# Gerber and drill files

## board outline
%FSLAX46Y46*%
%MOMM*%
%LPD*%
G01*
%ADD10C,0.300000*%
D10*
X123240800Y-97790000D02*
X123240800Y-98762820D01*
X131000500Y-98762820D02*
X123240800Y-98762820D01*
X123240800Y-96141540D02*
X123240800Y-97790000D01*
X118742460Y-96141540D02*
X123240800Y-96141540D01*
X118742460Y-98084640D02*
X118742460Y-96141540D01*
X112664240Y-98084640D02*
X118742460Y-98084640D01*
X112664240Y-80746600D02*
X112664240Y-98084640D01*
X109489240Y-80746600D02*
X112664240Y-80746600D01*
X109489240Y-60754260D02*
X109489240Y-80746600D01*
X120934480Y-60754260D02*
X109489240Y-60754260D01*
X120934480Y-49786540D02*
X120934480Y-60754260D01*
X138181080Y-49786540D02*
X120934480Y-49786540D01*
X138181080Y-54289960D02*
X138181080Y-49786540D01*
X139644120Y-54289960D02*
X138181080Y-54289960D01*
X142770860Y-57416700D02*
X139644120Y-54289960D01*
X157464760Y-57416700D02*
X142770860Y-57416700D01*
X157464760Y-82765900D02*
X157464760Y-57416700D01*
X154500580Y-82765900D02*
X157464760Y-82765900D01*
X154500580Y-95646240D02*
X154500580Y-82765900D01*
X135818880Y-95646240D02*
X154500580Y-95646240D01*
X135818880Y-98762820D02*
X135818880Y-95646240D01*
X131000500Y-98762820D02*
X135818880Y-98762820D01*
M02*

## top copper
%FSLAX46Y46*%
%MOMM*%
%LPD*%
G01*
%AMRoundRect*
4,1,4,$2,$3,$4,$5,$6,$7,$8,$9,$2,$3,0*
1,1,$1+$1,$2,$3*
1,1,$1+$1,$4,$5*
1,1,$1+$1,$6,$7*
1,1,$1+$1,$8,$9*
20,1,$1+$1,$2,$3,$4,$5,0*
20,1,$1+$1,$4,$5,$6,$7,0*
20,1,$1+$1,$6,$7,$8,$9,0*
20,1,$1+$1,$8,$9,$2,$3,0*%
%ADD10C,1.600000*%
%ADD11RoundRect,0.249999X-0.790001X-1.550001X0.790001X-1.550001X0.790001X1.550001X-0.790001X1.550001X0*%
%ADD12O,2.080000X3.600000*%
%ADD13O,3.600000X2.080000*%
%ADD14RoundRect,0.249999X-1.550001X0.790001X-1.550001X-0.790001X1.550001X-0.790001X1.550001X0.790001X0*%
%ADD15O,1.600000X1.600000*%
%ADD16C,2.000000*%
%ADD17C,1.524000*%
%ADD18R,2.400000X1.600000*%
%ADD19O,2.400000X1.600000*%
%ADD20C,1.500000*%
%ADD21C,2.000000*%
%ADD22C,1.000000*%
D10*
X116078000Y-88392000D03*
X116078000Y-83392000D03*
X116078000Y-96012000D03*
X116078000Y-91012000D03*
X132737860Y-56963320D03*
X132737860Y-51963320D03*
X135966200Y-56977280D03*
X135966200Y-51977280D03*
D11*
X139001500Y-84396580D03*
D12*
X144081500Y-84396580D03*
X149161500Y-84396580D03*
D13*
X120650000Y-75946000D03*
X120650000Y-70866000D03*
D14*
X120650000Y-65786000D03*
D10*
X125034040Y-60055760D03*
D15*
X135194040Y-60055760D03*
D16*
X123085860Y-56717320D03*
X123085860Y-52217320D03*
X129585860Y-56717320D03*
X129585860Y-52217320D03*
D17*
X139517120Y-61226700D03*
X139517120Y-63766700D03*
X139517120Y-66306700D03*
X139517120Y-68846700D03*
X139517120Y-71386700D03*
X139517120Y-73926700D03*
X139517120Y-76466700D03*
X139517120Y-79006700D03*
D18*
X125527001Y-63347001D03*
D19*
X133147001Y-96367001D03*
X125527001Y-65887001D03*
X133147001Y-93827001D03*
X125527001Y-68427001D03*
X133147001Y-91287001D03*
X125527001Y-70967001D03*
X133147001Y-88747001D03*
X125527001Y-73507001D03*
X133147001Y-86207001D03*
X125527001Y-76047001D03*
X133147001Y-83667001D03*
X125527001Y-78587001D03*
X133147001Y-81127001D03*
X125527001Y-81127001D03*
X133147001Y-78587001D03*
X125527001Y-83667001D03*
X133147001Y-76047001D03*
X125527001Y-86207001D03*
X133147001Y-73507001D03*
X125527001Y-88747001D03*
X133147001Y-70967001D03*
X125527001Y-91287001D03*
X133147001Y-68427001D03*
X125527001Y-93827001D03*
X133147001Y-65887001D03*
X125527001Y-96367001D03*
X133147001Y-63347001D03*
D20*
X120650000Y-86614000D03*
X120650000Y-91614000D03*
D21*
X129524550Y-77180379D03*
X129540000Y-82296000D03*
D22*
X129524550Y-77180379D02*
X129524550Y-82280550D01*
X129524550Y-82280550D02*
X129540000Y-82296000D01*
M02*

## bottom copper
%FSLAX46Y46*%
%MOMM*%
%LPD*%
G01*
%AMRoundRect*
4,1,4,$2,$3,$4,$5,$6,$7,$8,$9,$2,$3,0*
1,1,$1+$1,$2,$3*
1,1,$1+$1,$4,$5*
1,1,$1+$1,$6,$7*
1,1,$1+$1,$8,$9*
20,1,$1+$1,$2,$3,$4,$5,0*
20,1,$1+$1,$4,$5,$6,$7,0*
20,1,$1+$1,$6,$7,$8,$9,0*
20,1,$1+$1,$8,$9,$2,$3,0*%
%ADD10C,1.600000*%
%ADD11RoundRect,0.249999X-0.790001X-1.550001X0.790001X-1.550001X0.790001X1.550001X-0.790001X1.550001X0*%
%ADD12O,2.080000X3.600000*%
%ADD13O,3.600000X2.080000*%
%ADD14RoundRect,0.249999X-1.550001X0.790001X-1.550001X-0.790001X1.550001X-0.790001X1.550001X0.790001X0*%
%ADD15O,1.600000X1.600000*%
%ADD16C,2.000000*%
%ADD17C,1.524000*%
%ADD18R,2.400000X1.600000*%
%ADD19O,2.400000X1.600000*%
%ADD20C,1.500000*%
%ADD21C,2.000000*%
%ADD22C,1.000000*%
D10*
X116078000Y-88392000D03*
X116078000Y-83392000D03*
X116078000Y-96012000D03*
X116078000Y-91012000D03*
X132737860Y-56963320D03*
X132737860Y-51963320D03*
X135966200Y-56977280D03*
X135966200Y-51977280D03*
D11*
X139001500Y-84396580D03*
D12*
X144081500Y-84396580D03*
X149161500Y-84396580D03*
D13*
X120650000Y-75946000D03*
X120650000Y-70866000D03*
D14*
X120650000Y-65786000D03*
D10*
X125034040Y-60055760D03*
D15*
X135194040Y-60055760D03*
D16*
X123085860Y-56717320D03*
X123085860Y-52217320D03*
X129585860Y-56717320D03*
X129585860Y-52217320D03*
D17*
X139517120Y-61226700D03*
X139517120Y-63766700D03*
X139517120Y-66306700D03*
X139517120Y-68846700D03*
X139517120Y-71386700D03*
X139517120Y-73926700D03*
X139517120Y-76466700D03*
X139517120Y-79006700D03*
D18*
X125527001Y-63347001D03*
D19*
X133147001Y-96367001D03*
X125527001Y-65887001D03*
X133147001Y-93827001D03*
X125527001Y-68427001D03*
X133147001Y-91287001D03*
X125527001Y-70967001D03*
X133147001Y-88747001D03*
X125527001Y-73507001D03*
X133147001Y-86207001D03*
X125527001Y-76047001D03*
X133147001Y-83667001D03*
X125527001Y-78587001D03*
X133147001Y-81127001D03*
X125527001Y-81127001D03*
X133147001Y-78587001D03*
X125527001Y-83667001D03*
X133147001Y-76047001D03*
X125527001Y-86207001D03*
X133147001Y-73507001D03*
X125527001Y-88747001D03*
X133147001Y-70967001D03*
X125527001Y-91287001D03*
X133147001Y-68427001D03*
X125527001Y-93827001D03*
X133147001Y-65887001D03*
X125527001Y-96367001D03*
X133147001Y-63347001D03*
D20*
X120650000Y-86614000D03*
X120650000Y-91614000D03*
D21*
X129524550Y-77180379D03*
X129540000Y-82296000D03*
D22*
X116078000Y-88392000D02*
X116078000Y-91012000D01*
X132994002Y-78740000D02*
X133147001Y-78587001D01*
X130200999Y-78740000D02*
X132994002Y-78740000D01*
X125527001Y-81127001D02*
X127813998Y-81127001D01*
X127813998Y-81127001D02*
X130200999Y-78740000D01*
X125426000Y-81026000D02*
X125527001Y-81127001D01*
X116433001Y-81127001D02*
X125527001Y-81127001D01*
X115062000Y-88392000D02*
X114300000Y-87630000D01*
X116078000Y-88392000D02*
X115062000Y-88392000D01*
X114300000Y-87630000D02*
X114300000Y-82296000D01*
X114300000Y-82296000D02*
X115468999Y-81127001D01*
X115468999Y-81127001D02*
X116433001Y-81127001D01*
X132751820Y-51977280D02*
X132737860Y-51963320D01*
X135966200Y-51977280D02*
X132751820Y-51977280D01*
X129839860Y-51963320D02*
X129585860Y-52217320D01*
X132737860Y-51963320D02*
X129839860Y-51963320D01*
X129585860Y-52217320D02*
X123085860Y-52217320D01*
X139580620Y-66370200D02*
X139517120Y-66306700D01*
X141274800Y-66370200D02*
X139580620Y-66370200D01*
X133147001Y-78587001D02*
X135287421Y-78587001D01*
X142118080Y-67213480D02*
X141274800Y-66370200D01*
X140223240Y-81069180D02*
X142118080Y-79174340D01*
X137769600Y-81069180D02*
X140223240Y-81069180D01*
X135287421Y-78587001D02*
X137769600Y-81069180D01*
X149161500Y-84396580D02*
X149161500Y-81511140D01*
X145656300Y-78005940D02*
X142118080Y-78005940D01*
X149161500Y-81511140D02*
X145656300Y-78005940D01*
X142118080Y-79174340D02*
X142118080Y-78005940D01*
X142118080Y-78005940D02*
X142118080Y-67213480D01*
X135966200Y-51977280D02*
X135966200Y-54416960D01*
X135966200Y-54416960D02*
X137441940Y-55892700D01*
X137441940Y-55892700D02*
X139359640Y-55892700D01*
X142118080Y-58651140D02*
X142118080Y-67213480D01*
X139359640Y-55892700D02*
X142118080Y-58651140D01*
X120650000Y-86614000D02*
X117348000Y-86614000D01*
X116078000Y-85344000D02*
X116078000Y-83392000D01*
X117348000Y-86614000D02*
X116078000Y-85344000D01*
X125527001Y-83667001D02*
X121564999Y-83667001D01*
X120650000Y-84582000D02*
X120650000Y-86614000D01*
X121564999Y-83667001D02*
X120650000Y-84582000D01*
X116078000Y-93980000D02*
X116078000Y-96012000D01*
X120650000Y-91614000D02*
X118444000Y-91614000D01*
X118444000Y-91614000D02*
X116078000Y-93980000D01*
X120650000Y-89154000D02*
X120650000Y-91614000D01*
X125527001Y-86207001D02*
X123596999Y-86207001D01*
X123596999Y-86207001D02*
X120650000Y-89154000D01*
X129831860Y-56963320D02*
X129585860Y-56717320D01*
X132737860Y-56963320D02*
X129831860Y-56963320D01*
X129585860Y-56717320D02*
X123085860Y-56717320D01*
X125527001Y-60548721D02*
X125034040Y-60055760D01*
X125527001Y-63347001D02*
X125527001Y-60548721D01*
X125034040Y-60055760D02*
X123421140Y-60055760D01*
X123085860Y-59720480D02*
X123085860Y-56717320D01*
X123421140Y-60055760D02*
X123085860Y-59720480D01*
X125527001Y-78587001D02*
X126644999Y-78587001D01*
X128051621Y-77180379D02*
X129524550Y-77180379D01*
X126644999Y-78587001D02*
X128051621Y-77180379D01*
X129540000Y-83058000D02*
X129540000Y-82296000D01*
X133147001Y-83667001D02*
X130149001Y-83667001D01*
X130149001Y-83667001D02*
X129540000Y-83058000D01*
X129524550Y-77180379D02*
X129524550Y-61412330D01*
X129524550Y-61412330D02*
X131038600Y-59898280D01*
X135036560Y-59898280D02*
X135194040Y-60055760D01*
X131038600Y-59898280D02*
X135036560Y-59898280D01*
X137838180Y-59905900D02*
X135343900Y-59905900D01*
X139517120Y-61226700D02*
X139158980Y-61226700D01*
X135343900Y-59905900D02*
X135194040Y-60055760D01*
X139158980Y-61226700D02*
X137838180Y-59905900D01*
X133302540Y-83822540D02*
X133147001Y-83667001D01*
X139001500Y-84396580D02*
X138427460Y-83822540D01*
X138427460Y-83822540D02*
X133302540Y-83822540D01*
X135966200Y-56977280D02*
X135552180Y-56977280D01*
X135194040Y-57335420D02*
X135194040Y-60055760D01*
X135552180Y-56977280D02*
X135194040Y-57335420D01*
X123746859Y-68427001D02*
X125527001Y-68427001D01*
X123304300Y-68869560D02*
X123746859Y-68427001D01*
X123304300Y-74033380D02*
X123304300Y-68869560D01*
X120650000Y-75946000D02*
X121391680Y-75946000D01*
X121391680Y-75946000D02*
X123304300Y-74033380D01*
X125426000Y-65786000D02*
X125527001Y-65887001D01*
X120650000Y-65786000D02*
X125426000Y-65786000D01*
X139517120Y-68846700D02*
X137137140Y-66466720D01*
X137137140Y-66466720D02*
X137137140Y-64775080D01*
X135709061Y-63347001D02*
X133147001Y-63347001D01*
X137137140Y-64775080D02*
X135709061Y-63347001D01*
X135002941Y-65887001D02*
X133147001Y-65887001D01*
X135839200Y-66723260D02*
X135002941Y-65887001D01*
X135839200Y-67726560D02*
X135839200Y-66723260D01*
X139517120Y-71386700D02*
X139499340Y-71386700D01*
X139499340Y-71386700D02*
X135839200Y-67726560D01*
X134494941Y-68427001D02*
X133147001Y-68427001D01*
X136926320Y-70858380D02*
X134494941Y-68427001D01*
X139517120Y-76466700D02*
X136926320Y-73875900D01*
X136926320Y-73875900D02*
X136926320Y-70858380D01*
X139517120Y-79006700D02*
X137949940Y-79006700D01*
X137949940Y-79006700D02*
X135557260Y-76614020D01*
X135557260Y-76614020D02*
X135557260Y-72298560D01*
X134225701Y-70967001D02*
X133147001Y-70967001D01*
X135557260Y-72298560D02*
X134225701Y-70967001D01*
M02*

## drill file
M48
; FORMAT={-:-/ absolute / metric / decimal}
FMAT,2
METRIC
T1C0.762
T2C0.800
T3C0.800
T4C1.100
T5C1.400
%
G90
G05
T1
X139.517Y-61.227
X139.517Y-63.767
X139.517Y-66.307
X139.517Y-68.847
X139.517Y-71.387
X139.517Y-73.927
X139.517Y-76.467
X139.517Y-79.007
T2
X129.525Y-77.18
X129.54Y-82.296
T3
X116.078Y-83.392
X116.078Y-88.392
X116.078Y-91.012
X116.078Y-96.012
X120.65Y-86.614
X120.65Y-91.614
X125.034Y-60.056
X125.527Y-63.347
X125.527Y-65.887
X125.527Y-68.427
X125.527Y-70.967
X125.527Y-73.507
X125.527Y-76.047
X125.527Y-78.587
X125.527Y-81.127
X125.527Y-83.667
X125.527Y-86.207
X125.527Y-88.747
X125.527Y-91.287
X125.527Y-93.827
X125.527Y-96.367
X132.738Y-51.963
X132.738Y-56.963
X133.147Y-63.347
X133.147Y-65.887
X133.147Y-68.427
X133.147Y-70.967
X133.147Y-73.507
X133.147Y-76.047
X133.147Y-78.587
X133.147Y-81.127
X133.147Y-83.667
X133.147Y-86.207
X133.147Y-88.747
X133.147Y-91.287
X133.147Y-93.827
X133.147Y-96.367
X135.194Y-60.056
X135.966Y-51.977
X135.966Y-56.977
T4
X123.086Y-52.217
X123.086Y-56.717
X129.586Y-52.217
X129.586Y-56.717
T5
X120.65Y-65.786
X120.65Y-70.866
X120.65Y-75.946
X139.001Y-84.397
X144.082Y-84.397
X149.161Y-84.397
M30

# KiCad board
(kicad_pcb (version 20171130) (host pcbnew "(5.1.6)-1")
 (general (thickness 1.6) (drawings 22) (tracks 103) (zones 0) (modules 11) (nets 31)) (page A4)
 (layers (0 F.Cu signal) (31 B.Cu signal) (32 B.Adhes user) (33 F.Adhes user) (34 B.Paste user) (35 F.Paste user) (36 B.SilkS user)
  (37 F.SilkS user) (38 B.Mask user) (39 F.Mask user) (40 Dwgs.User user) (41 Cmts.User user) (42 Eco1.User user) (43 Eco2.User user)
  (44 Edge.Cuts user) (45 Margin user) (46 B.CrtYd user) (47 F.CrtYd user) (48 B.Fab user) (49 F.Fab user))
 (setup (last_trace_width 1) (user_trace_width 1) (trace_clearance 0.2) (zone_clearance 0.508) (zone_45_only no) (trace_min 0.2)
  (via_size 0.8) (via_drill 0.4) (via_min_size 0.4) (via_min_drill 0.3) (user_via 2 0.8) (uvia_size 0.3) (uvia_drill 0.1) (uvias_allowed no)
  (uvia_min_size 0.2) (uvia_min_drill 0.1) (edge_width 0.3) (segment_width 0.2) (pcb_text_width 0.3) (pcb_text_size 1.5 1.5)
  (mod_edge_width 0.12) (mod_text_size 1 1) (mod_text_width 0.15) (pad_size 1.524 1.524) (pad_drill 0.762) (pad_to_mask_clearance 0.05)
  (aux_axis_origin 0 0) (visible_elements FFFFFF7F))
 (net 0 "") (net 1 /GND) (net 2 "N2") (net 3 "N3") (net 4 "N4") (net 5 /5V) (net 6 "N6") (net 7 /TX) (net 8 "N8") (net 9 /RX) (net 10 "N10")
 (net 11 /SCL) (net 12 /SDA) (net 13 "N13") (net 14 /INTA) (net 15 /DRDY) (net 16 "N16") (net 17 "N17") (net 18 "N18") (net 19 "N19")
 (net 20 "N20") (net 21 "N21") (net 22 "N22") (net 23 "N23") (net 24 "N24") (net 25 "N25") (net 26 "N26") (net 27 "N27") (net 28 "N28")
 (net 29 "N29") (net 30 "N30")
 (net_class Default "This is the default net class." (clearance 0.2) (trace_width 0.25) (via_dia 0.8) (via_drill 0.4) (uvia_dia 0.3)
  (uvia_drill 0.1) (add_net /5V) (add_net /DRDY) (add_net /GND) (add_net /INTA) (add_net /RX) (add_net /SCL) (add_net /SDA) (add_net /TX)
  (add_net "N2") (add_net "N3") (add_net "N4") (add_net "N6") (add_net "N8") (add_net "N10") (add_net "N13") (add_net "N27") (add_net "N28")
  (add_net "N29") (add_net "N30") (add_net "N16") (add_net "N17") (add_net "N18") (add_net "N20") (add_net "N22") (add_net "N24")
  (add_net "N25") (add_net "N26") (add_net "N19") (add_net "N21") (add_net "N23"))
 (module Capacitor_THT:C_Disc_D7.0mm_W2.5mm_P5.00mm (layer F.Cu) (at 116.078 83.392 270)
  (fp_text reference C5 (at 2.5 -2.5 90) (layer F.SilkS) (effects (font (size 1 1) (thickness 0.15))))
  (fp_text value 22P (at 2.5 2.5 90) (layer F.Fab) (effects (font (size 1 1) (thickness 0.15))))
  (pad 2 thru_hole circle (at 5 0 270) (size 1.6 1.6) (drill 0.8) (layers *.Cu *.Mask) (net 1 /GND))
  (pad 1 thru_hole circle (at 0 0 270) (size 1.6 1.6) (drill 0.8) (layers *.Cu *.Mask) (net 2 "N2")))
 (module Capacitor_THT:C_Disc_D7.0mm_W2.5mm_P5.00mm (layer F.Cu) (at 116.078 96.012 90)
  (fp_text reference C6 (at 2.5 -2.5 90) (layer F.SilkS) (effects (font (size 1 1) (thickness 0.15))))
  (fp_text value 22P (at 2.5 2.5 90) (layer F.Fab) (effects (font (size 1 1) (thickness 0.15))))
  (pad 1 thru_hole circle (at 0 0 90) (size 1.6 1.6) (drill 0.8) (layers *.Cu *.Mask) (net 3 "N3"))
  (pad 2 thru_hole circle (at 5 0 90) (size 1.6 1.6) (drill 0.8) (layers *.Cu *.Mask) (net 1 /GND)))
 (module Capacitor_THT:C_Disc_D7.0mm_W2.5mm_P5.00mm (layer F.Cu) (at 132.73786 51.96332 270)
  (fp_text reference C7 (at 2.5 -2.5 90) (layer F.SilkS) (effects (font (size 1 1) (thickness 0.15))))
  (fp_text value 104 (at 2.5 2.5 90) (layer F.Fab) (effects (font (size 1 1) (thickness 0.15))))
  (pad 2 thru_hole circle (at 5 0 270) (size 1.6 1.6) (drill 0.8) (layers *.Cu *.Mask) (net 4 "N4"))
  (pad 1 thru_hole circle (at 0 0 270) (size 1.6 1.6) (drill 0.8) (layers *.Cu *.Mask) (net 1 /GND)))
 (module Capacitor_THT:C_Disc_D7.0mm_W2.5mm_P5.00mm (layer F.Cu) (at 135.9662 56.97728 90)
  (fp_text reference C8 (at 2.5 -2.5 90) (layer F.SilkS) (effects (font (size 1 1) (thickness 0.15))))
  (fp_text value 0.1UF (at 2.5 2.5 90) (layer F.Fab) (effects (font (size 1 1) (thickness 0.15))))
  (pad 1 thru_hole circle (at 0 0 90) (size 1.6 1.6) (drill 0.8) (layers *.Cu *.Mask) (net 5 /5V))
  (pad 2 thru_hole circle (at 5 0 90) (size 1.6 1.6) (drill 0.8) (layers *.Cu *.Mask) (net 1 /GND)))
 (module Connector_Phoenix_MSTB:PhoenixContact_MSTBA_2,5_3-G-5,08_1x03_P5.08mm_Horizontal (layer F.Cu) (at 139.0015 84.39658)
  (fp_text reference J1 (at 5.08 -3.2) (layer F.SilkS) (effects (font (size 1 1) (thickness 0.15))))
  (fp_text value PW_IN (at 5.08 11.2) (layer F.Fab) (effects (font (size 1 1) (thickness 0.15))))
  (pad 1 thru_hole roundrect (at 0 0) (size 2.08 3.6) (drill 1.4) (layers *.Cu *.Mask) (roundrect_rratio 0.120192) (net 5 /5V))
  (pad 2 thru_hole oval (at 5.08 0) (size 2.08 3.6) (drill 1.4) (layers *.Cu *.Mask) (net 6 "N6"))
  (pad 3 thru_hole oval (at 10.16 0) (size 2.08 3.6) (drill 1.4) (layers *.Cu *.Mask) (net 1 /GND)))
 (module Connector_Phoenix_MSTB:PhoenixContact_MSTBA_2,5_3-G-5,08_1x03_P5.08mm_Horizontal (layer F.Cu) (at 120.65 65.786 270)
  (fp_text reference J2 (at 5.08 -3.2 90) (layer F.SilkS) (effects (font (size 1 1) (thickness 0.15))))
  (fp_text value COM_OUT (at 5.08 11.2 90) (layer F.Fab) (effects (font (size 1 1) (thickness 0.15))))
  (pad 3 thru_hole oval (at 10.16 0 270) (size 2.08 3.6) (drill 1.4) (layers *.Cu *.Mask) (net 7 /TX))
  (pad 2 thru_hole oval (at 5.08 0 270) (size 2.08 3.6) (drill 1.4) (layers *.Cu *.Mask) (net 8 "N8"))
  (pad 1 thru_hole roundrect (at 0 0 270) (size 2.08 3.6) (drill 1.4) (layers *.Cu *.Mask) (roundrect_rratio 0.120192) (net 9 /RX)))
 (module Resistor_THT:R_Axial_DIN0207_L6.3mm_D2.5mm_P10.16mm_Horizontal (layer F.Cu) (at 125.03404 60.05576)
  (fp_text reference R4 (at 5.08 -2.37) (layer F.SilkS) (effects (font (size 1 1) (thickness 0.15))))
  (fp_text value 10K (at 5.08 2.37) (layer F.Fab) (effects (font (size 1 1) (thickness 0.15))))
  (pad 1 thru_hole circle (at 0 0) (size 1.6 1.6) (drill 0.8) (layers *.Cu *.Mask) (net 4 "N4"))
  (pad 2 thru_hole oval (at 10.16 0) (size 1.6 1.6) (drill 0.8) (layers *.Cu *.Mask) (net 5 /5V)))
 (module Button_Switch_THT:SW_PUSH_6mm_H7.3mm (layer F.Cu) (at 123.08586 52.21732)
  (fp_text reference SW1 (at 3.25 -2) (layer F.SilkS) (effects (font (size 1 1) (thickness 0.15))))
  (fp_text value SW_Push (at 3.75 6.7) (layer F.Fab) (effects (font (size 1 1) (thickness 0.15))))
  (pad 2 thru_hole circle (at 0 4.5 90) (size 2 2) (drill 1.1) (layers *.Cu *.Mask) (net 4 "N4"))
  (pad 1 thru_hole circle (at 0 0 90) (size 2 2) (drill 1.1) (layers *.Cu *.Mask) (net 1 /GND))
  (pad 2 thru_hole circle (at 6.5 4.5 90) (size 2 2) (drill 1.1) (layers *.Cu *.Mask) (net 4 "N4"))
  (pad 1 thru_hole circle (at 6.5 0 90) (size 2 2) (drill 1.1) (layers *.Cu *.Mask) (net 1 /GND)))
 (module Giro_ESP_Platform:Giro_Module (layer F.Cu) (at 139.51712 57.4167)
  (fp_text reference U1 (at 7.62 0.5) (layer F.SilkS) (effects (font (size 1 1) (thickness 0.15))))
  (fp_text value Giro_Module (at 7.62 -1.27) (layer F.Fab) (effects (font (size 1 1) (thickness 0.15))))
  (pad 1 thru_hole circle (at 0 3.81) (size 1.524 1.524) (drill 0.762) (layers *.Cu *.Mask) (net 5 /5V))
  (pad 2 thru_hole circle (at 0 6.35) (size 1.524 1.524) (drill 0.762) (layers *.Cu *.Mask) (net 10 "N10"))
  (pad 3 thru_hole circle (at 0 8.89) (size 1.524 1.524) (drill 0.762) (layers *.Cu *.Mask) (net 1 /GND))
  (pad 4 thru_hole circle (at 0 11.43) (size 1.524 1.524) (drill 0.762) (layers *.Cu *.Mask) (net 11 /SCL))
  (pad 5 thru_hole circle (at 0 13.97) (size 1.524 1.524) (drill 0.762) (layers *.Cu *.Mask) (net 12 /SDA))
  (pad 6 thru_hole circle (at 0 16.51) (size 1.524 1.524) (drill 0.762) (layers *.Cu *.Mask) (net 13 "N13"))
  (pad 7 thru_hole circle (at 0 19.05) (size 1.524 1.524) (drill 0.762) (layers *.Cu *.Mask) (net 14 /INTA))
  (pad 8 thru_hole circle (at 0 21.59) (size 1.524 1.524) (drill 0.762) (layers *.Cu *.Mask) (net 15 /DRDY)))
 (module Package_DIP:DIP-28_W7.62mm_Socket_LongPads (layer F.Cu) (at 125.527001 63.347001)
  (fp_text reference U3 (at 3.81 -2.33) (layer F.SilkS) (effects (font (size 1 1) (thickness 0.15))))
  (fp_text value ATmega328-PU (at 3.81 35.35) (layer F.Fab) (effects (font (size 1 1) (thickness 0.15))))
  (pad 1 thru_hole rect (at 0 0) (size 2.4 1.6) (drill 0.8) (layers *.Cu *.Mask) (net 4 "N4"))
  (pad 15 thru_hole oval (at 7.62 33.02) (size 2.4 1.6) (drill 0.8) (layers *.Cu *.Mask) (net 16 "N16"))
  (pad 2 thru_hole oval (at 0 2.54) (size 2.4 1.6) (drill 0.8) (layers *.Cu *.Mask) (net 9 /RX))
  (pad 16 thru_hole oval (at 7.62 30.48) (size 2.4 1.6) (drill 0.8) (layers *.Cu *.Mask) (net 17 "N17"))
  (pad 3 thru_hole oval (at 0 5.08) (size 2.4 1.6) (drill 0.8) (layers *.Cu *.Mask) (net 7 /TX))
  (pad 17 thru_hole oval (at 7.62 27.94) (size 2.4 1.6) (drill 0.8) (layers *.Cu *.Mask) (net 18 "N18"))
  (pad 4 thru_hole oval (at 0 7.62) (size 2.4 1.6) (drill 0.8) (layers *.Cu *.Mask) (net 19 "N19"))
  (pad 18 thru_hole oval (at 7.62 25.4) (size 2.4 1.6) (drill 0.8) (layers *.Cu *.Mask) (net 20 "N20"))
  (pad 5 thru_hole oval (at 0 10.16) (size 2.4 1.6) (drill 0.8) (layers *.Cu *.Mask) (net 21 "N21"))
  (pad 19 thru_hole oval (at 7.62 22.86) (size 2.4 1.6) (drill 0.8) (layers *.Cu *.Mask) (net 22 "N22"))
  (pad 6 thru_hole oval (at 0 12.7) (size 2.4 1.6) (drill 0.8) (layers *.Cu *.Mask) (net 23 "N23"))
  (pad 20 thru_hole oval (at 7.62 20.32) (size 2.4 1.6) (drill 0.8) (layers *.Cu *.Mask) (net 5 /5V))
  (pad 7 thru_hole oval (at 0 15.24) (size 2.4 1.6) (drill 0.8) (layers *.Cu *.Mask) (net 5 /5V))
  (pad 21 thru_hole oval (at 7.62 17.78) (size 2.4 1.6) (drill 0.8) (layers *.Cu *.Mask) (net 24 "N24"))
  (pad 8 thru_hole oval (at 0 17.78) (size 2.4 1.6) (drill 0.8) (layers *.Cu *.Mask) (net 1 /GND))
  (pad 22 thru_hole oval (at 7.62 15.24) (size 2.4 1.6) (drill 0.8) (layers *.Cu *.Mask) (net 1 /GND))
  (pad 9 thru_hole oval (at 0 20.32) (size 2.4 1.6) (drill 0.8) (layers *.Cu *.Mask) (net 2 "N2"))
  (pad 23 thru_hole oval (at 7.62 12.7) (size 2.4 1.6) (drill 0.8) (layers *.Cu *.Mask) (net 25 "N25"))
  (pad 10 thru_hole oval (at 0 22.86) (size 2.4 1.6) (drill 0.8) (layers *.Cu *.Mask) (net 3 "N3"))
  (pad 24 thru_hole oval (at 7.62 10.16) (size 2.4 1.6) (drill 0.8) (layers *.Cu *.Mask) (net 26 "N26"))
  (pad 11 thru_hole oval (at 0 25.4) (size 2.4 1.6) (drill 0.8) (layers *.Cu *.Mask) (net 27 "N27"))
  (pad 25 thru_hole oval (at 7.62 7.62) (size 2.4 1.6) (drill 0.8) (layers *.Cu *.Mask) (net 15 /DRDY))
  (pad 12 thru_hole oval (at 0 27.94) (size 2.4 1.6) (drill 0.8) (layers *.Cu *.Mask) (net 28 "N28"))
  (pad 26 thru_hole oval (at 7.62 5.08) (size 2.4 1.6) (drill 0.8) (layers *.Cu *.Mask) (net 14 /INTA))
  (pad 13 thru_hole oval (at 0 30.48) (size 2.4 1.6) (drill 0.8) (layers *.Cu *.Mask) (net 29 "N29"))
  (pad 27 thru_hole oval (at 7.62 2.54) (size 2.4 1.6) (drill 0.8) (layers *.Cu *.Mask) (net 12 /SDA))
  (pad 14 thru_hole oval (at 0 33.02) (size 2.4 1.6) (drill 0.8) (layers *.Cu *.Mask) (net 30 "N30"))
  (pad 28 thru_hole oval (at 7.62 0) (size 2.4 1.6) (drill 0.8) (layers *.Cu *.Mask) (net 11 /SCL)))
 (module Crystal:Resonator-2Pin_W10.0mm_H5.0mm (layer F.Cu) (at 120.65 86.614 270)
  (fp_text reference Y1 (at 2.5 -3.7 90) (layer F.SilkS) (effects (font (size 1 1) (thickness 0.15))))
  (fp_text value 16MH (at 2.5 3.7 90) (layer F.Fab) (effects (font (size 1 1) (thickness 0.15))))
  (pad 1 thru_hole circle (at 0 0 270) (size 1.5 1.5) (drill 0.8) (layers *.Cu *.Mask) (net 2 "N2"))
  (pad 2 thru_hole circle (at 5 0 270) (size 1.5 1.5) (drill 0.8) (layers *.Cu *.Mask) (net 3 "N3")))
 (gr_line (start 123.2408 97.79) (end 123.2408 98.76282) (layer Edge.Cuts) (width 0.3))
 (gr_line (start 131.0005 98.76282) (end 123.2408 98.76282) (layer Edge.Cuts) (width 0.3))
 (gr_line (start 123.2408 96.14154) (end 123.2408 97.79) (layer Edge.Cuts) (width 0.3))
 (gr_line (start 118.74246 96.14154) (end 123.2408 96.14154) (layer Edge.Cuts) (width 0.3))
 (gr_line (start 118.74246 98.08464) (end 118.74246 96.14154) (layer Edge.Cuts) (width 0.3))
 (gr_line (start 112.66424 98.08464) (end 118.74246 98.08464) (layer Edge.Cuts) (width 0.3))
 (gr_line (start 112.66424 80.7466) (end 112.66424 98.08464) (layer Edge.Cuts) (width 0.3))
 (gr_line (start 109.48924 80.7466) (end 112.66424 80.7466) (layer Edge.Cuts) (width 0.3))
 (gr_line (start 109.48924 60.75426) (end 109.48924 80.7466) (layer Edge.Cuts) (width 0.3))
 (gr_line (start 120.93448 60.75426) (end 109.48924 60.75426) (layer Edge.Cuts) (width 0.3))
 (gr_line (start 120.93448 49.78654) (end 120.93448 60.75426) (layer Edge.Cuts) (width 0.3))
 (gr_line (start 138.18108 49.78654) (end 120.93448 49.78654) (layer Edge.Cuts) (width 0.3))
 (gr_line (start 138.18108 54.28996) (end 138.18108 49.78654) (layer Edge.Cuts) (width 0.3))
 (gr_line (start 139.64412 54.28996) (end 138.18108 54.28996) (layer Edge.Cuts) (width 0.3))
 (gr_line (start 142.77086 57.4167) (end 139.64412 54.28996) (layer Edge.Cuts) (width 0.3))
 (gr_line (start 157.46476 57.4167) (end 142.77086 57.4167) (layer Edge.Cuts) (width 0.3))
 (gr_line (start 157.46476 82.7659) (end 157.46476 57.4167) (layer Edge.Cuts) (width 0.3))
 (gr_line (start 154.50058 82.7659) (end 157.46476 82.7659) (layer Edge.Cuts) (width 0.3))
 (gr_line (start 154.50058 95.64624) (end 154.50058 82.7659) (layer Edge.Cuts) (width 0.3))
 (gr_line (start 135.81888 95.64624) (end 154.50058 95.64624) (layer Edge.Cuts) (width 0.3))
 (gr_line (start 135.81888 98.76282) (end 135.81888 95.64624) (layer Edge.Cuts) (width 0.3))
 (gr_line (start 131.0005 98.76282) (end 135.81888 98.76282) (layer Edge.Cuts) (width 0.3))
 (segment (start 116.078 88.392) (end 116.078 91.012) (width 1) (layer B.Cu) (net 1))
 (segment (start 132.994002 78.74) (end 133.147001 78.587001) (width 1) (layer B.Cu) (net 1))
 (segment (start 130.200999 78.74) (end 132.994002 78.74) (width 1) (layer B.Cu) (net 1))
 (segment (start 125.527001 81.127001) (end 127.813998 81.127001) (width 1) (layer B.Cu) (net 1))
 (segment (start 127.813998 81.127001) (end 130.200999 78.74) (width 1) (layer B.Cu) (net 1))
 (segment (start 125.426 81.026) (end 125.527001 81.127001) (width 1) (layer B.Cu) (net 1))
 (segment (start 116.433001 81.127001) (end 125.527001 81.127001) (width 1) (layer B.Cu) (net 1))
 (segment (start 115.062 88.392) (end 114.3 87.63) (width 1) (layer B.Cu) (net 1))
 (segment (start 116.078 88.392) (end 115.062 88.392) (width 1) (layer B.Cu) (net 1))
 (segment (start 114.3 87.63) (end 114.3 82.296) (width 1) (layer B.Cu) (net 1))
 (segment (start 114.3 82.296) (end 115.468999 81.127001) (width 1) (layer B.Cu) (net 1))
 (segment (start 115.468999 81.127001) (end 116.433001 81.127001) (width 1) (layer B.Cu) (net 1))
 (segment (start 132.75182 51.97728) (end 132.73786 51.96332) (width 1) (layer B.Cu) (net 1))
 (segment (start 135.9662 51.97728) (end 132.75182 51.97728) (width 1) (layer B.Cu) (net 1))
 (segment (start 129.83986 51.96332) (end 129.58586 52.21732) (width 1) (layer B.Cu) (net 1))
 (segment (start 132.73786 51.96332) (end 129.83986 51.96332) (width 1) (layer B.Cu) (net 1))
 (segment (start 129.58586 52.21732) (end 123.08586 52.21732) (width 1) (layer B.Cu) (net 1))
 (segment (start 139.58062 66.3702) (end 139.51712 66.3067) (width 1) (layer B.Cu) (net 1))
 (segment (start 141.2748 66.3702) (end 139.58062 66.3702) (width 1) (layer B.Cu) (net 1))
 (segment (start 133.147001 78.587001) (end 135.287421 78.587001) (width 1) (layer B.Cu) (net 1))
 (segment (start 142.11808 67.21348) (end 141.2748 66.3702) (width 1) (layer B.Cu) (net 1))
 (segment (start 140.22324 81.06918) (end 142.11808 79.17434) (width 1) (layer B.Cu) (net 1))
 (segment (start 137.7696 81.06918) (end 140.22324 81.06918) (width 1) (layer B.Cu) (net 1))
 (segment (start 135.287421 78.587001) (end 137.7696 81.06918) (width 1) (layer B.Cu) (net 1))
 (segment (start 149.1615 84.39658) (end 149.1615 81.51114) (width 1) (layer B.Cu) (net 1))
 (segment (start 145.6563 78.00594) (end 142.11808 78.00594) (width 1) (layer B.Cu) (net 1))
 (segment (start 149.1615 81.51114) (end 145.6563 78.00594) (width 1) (layer B.Cu) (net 1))
 (segment (start 142.11808 79.17434) (end 142.11808 78.00594) (width 1) (layer B.Cu) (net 1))
 (segment (start 142.11808 78.00594) (end 142.11808 67.21348) (width 1) (layer B.Cu) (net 1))
 (segment (start 135.9662 51.97728) (end 135.9662 54.41696) (width 1) (layer B.Cu) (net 1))
 (segment (start 135.9662 54.41696) (end 137.44194 55.8927) (width 1) (layer B.Cu) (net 1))
 (segment (start 137.44194 55.8927) (end 139.35964 55.8927) (width 1) (layer B.Cu) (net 1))
 (segment (start 142.11808 58.65114) (end 142.11808 67.21348) (width 1) (layer B.Cu) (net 1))
 (segment (start 139.35964 55.8927) (end 142.11808 58.65114) (width 1) (layer B.Cu) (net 1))
 (segment (start 120.65 86.614) (end 117.348 86.614) (width 1) (layer B.Cu) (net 2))
 (segment (start 116.078 85.344) (end 116.078 83.392) (width 1) (layer B.Cu) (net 2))
 (segment (start 117.348 86.614) (end 116.078 85.344) (width 1) (layer B.Cu) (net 2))
 (segment (start 125.527001 83.667001) (end 121.564999 83.667001) (width 1) (layer B.Cu) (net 2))
 (segment (start 120.65 84.582) (end 120.65 86.614) (width 1) (layer B.Cu) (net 2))
 (segment (start 121.564999 83.667001) (end 120.65 84.582) (width 1) (layer B.Cu) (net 2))
 (segment (start 116.078 93.98) (end 116.078 96.012) (width 1) (layer B.Cu) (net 3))
 (segment (start 120.65 91.614) (end 118.444 91.614) (width 1) (layer B.Cu) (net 3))
 (segment (start 118.444 91.614) (end 116.078 93.98) (width 1) (layer B.Cu) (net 3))
 (segment (start 120.65 89.154) (end 120.65 91.614) (width 1) (layer B.Cu) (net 3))
 (segment (start 125.527001 86.207001) (end 123.596999 86.207001) (width 1) (layer B.Cu) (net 3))
 (segment (start 123.596999 86.207001) (end 120.65 89.154) (width 1) (layer B.Cu) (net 3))
 (segment (start 129.83186 56.96332) (end 129.58586 56.71732) (width 1) (layer B.Cu) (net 4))
 (segment (start 132.73786 56.96332) (end 129.83186 56.96332) (width 1) (layer B.Cu) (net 4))
 (segment (start 129.58586 56.71732) (end 123.08586 56.71732) (width 1) (layer B.Cu) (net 4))
 (segment (start 125.527001 60.548721) (end 125.03404 60.05576) (width 1) (layer B.Cu) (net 4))
 (segment (start 125.527001 63.347001) (end 125.527001 60.548721) (width 1) (layer B.Cu) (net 4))
 (segment (start 125.03404 60.05576) (end 123.42114 60.05576) (width 1) (layer B.Cu) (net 4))
 (segment (start 123.08586 59.72048) (end 123.08586 56.71732) (width 1) (layer B.Cu) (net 4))
 (segment (start 123.42114 60.05576) (end 123.08586 59.72048) (width 1) (layer B.Cu) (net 4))
 (via (at 129.52455 77.180379) (size 2) (drill 0.8) (layers F.Cu B.Cu) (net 5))
 (segment (start 125.527001 78.587001) (end 126.644999 78.587001) (width 1) (layer B.Cu) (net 5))
 (segment (start 128.051621 77.180379) (end 129.52455 77.180379) (width 1) (layer B.Cu) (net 5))
 (segment (start 126.644999 78.587001) (end 128.051621 77.180379) (width 1) (layer B.Cu) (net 5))
 (via (at 129.54 82.296) (size 2) (drill 0.8) (layers F.Cu B.Cu) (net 5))
 (segment (start 129.52455 77.180379) (end 129.52455 82.28055) (width 1) (layer F.Cu) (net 5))
 (segment (start 129.52455 82.28055) (end 129.54 82.296) (width 1) (layer F.Cu) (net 5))
 (segment (start 129.54 83.058) (end 129.54 82.296) (width 1) (layer B.Cu) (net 5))
 (segment (start 133.147001 83.667001) (end 130.149001 83.667001) (width 1) (layer B.Cu) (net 5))
 (segment (start 130.149001 83.667001) (end 129.54 83.058) (width 1) (layer B.Cu) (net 5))
 (segment (start 129.52455 77.180379) (end 129.52455 61.41233) (width 1) (layer B.Cu) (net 5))
 (segment (start 129.52455 61.41233) (end 131.0386 59.89828) (width 1) (layer B.Cu) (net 5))
 (segment (start 135.03656 59.89828) (end 135.19404 60.05576) (width 1) (layer B.Cu) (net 5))
 (segment (start 131.0386 59.89828) (end 135.03656 59.89828) (width 1) (layer B.Cu) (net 5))
 (segment (start 137.83818 59.9059) (end 135.3439 59.9059) (width 1) (layer B.Cu) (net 5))
 (segment (start 139.51712 61.2267) (end 139.15898 61.2267) (width 1) (layer B.Cu) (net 5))
 (segment (start 135.3439 59.9059) (end 135.19404 60.05576) (width 1) (layer B.Cu) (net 5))
 (segment (start 139.15898 61.2267) (end 137.83818 59.9059) (width 1) (layer B.Cu) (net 5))
 (segment (start 133.30254 83.82254) (end 133.147001 83.667001) (width 1) (layer B.Cu) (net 5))
 (segment (start 139.0015 84.39658) (end 138.42746 83.82254) (width 1) (layer B.Cu) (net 5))
 (segment (start 138.42746 83.82254) (end 133.30254 83.82254) (width 1) (layer B.Cu) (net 5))
 (segment (start 135.9662 56.97728) (end 135.55218 56.97728) (width 1) (layer B.Cu) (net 5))
 (segment (start 135.19404 57.33542) (end 135.19404 60.05576) (width 1) (layer B.Cu) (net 5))
 (segment (start 135.55218 56.97728) (end 135.19404 57.33542) (width 1) (layer B.Cu) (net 5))
 (segment (start 123.746859 68.427001) (end 125.527001 68.427001) (width 1) (layer B.Cu) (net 7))
 (segment (start 123.3043 68.86956) (end 123.746859 68.427001) (width 1) (layer B.Cu) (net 7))
 (segment (start 123.3043 74.03338) (end 123.3043 68.86956) (width 1) (layer B.Cu) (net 7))
 (segment (start 120.65 75.946) (end 121.39168 75.946) (width 1) (layer B.Cu) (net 7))
 (segment (start 121.39168 75.946) (end 123.3043 74.03338) (width 1) (layer B.Cu) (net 7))
 (segment (start 125.426 65.786) (end 125.527001 65.887001) (width 1) (layer B.Cu) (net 9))
 (segment (start 120.65 65.786) (end 125.426 65.786) (width 1) (layer B.Cu) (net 9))
 (segment (start 139.51712 68.8467) (end 137.13714 66.46672) (width 1) (layer B.Cu) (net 11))
 (segment (start 137.13714 66.46672) (end 137.13714 64.77508) (width 1) (layer B.Cu) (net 11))
 (segment (start 135.709061 63.347001) (end 133.147001 63.347001) (width 1) (layer B.Cu) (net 11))
 (segment (start 137.13714 64.77508) (end 135.709061 63.347001) (width 1) (layer B.Cu) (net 11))
 (segment (start 135.002941 65.887001) (end 133.147001 65.887001) (width 1) (layer B.Cu) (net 12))
 (segment (start 135.8392 66.72326) (end 135.002941 65.887001) (width 1) (layer B.Cu) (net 12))
 (segment (start 135.8392 67.72656) (end 135.8392 66.72326) (width 1) (layer B.Cu) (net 12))
 (segment (start 139.51712 71.3867) (end 139.49934 71.3867) (width 1) (layer B.Cu) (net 12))
 (segment (start 139.49934 71.3867) (end 135.8392 67.72656) (width 1) (layer B.Cu) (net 12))
 (segment (start 134.494941 68.427001) (end 133.147001 68.427001) (width 1) (layer B.Cu) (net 14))
 (segment (start 136.92632 70.85838) (end 134.494941 68.427001) (width 1) (layer B.Cu) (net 14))
 (segment (start 139.51712 76.4667) (end 136.92632 73.8759) (width 1) (layer B.Cu) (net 14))
 (segment (start 136.92632 73.8759) (end 136.92632 70.85838) (width 1) (layer B.Cu) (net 14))
 (segment (start 139.51712 79.0067) (end 137.94994 79.0067) (width 1) (layer B.Cu) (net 15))
 (segment (start 137.94994 79.0067) (end 135.55726 76.61402) (width 1) (layer B.Cu) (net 15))
 (segment (start 135.55726 76.61402) (end 135.55726 72.29856) (width 1) (layer B.Cu) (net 15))
 (segment (start 134.225701 70.967001) (end 133.147001 70.967001) (width 1) (layer B.Cu) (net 15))
 (segment (start 135.55726 72.29856) (end 134.225701 70.967001) (width 1) (layer B.Cu) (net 15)))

